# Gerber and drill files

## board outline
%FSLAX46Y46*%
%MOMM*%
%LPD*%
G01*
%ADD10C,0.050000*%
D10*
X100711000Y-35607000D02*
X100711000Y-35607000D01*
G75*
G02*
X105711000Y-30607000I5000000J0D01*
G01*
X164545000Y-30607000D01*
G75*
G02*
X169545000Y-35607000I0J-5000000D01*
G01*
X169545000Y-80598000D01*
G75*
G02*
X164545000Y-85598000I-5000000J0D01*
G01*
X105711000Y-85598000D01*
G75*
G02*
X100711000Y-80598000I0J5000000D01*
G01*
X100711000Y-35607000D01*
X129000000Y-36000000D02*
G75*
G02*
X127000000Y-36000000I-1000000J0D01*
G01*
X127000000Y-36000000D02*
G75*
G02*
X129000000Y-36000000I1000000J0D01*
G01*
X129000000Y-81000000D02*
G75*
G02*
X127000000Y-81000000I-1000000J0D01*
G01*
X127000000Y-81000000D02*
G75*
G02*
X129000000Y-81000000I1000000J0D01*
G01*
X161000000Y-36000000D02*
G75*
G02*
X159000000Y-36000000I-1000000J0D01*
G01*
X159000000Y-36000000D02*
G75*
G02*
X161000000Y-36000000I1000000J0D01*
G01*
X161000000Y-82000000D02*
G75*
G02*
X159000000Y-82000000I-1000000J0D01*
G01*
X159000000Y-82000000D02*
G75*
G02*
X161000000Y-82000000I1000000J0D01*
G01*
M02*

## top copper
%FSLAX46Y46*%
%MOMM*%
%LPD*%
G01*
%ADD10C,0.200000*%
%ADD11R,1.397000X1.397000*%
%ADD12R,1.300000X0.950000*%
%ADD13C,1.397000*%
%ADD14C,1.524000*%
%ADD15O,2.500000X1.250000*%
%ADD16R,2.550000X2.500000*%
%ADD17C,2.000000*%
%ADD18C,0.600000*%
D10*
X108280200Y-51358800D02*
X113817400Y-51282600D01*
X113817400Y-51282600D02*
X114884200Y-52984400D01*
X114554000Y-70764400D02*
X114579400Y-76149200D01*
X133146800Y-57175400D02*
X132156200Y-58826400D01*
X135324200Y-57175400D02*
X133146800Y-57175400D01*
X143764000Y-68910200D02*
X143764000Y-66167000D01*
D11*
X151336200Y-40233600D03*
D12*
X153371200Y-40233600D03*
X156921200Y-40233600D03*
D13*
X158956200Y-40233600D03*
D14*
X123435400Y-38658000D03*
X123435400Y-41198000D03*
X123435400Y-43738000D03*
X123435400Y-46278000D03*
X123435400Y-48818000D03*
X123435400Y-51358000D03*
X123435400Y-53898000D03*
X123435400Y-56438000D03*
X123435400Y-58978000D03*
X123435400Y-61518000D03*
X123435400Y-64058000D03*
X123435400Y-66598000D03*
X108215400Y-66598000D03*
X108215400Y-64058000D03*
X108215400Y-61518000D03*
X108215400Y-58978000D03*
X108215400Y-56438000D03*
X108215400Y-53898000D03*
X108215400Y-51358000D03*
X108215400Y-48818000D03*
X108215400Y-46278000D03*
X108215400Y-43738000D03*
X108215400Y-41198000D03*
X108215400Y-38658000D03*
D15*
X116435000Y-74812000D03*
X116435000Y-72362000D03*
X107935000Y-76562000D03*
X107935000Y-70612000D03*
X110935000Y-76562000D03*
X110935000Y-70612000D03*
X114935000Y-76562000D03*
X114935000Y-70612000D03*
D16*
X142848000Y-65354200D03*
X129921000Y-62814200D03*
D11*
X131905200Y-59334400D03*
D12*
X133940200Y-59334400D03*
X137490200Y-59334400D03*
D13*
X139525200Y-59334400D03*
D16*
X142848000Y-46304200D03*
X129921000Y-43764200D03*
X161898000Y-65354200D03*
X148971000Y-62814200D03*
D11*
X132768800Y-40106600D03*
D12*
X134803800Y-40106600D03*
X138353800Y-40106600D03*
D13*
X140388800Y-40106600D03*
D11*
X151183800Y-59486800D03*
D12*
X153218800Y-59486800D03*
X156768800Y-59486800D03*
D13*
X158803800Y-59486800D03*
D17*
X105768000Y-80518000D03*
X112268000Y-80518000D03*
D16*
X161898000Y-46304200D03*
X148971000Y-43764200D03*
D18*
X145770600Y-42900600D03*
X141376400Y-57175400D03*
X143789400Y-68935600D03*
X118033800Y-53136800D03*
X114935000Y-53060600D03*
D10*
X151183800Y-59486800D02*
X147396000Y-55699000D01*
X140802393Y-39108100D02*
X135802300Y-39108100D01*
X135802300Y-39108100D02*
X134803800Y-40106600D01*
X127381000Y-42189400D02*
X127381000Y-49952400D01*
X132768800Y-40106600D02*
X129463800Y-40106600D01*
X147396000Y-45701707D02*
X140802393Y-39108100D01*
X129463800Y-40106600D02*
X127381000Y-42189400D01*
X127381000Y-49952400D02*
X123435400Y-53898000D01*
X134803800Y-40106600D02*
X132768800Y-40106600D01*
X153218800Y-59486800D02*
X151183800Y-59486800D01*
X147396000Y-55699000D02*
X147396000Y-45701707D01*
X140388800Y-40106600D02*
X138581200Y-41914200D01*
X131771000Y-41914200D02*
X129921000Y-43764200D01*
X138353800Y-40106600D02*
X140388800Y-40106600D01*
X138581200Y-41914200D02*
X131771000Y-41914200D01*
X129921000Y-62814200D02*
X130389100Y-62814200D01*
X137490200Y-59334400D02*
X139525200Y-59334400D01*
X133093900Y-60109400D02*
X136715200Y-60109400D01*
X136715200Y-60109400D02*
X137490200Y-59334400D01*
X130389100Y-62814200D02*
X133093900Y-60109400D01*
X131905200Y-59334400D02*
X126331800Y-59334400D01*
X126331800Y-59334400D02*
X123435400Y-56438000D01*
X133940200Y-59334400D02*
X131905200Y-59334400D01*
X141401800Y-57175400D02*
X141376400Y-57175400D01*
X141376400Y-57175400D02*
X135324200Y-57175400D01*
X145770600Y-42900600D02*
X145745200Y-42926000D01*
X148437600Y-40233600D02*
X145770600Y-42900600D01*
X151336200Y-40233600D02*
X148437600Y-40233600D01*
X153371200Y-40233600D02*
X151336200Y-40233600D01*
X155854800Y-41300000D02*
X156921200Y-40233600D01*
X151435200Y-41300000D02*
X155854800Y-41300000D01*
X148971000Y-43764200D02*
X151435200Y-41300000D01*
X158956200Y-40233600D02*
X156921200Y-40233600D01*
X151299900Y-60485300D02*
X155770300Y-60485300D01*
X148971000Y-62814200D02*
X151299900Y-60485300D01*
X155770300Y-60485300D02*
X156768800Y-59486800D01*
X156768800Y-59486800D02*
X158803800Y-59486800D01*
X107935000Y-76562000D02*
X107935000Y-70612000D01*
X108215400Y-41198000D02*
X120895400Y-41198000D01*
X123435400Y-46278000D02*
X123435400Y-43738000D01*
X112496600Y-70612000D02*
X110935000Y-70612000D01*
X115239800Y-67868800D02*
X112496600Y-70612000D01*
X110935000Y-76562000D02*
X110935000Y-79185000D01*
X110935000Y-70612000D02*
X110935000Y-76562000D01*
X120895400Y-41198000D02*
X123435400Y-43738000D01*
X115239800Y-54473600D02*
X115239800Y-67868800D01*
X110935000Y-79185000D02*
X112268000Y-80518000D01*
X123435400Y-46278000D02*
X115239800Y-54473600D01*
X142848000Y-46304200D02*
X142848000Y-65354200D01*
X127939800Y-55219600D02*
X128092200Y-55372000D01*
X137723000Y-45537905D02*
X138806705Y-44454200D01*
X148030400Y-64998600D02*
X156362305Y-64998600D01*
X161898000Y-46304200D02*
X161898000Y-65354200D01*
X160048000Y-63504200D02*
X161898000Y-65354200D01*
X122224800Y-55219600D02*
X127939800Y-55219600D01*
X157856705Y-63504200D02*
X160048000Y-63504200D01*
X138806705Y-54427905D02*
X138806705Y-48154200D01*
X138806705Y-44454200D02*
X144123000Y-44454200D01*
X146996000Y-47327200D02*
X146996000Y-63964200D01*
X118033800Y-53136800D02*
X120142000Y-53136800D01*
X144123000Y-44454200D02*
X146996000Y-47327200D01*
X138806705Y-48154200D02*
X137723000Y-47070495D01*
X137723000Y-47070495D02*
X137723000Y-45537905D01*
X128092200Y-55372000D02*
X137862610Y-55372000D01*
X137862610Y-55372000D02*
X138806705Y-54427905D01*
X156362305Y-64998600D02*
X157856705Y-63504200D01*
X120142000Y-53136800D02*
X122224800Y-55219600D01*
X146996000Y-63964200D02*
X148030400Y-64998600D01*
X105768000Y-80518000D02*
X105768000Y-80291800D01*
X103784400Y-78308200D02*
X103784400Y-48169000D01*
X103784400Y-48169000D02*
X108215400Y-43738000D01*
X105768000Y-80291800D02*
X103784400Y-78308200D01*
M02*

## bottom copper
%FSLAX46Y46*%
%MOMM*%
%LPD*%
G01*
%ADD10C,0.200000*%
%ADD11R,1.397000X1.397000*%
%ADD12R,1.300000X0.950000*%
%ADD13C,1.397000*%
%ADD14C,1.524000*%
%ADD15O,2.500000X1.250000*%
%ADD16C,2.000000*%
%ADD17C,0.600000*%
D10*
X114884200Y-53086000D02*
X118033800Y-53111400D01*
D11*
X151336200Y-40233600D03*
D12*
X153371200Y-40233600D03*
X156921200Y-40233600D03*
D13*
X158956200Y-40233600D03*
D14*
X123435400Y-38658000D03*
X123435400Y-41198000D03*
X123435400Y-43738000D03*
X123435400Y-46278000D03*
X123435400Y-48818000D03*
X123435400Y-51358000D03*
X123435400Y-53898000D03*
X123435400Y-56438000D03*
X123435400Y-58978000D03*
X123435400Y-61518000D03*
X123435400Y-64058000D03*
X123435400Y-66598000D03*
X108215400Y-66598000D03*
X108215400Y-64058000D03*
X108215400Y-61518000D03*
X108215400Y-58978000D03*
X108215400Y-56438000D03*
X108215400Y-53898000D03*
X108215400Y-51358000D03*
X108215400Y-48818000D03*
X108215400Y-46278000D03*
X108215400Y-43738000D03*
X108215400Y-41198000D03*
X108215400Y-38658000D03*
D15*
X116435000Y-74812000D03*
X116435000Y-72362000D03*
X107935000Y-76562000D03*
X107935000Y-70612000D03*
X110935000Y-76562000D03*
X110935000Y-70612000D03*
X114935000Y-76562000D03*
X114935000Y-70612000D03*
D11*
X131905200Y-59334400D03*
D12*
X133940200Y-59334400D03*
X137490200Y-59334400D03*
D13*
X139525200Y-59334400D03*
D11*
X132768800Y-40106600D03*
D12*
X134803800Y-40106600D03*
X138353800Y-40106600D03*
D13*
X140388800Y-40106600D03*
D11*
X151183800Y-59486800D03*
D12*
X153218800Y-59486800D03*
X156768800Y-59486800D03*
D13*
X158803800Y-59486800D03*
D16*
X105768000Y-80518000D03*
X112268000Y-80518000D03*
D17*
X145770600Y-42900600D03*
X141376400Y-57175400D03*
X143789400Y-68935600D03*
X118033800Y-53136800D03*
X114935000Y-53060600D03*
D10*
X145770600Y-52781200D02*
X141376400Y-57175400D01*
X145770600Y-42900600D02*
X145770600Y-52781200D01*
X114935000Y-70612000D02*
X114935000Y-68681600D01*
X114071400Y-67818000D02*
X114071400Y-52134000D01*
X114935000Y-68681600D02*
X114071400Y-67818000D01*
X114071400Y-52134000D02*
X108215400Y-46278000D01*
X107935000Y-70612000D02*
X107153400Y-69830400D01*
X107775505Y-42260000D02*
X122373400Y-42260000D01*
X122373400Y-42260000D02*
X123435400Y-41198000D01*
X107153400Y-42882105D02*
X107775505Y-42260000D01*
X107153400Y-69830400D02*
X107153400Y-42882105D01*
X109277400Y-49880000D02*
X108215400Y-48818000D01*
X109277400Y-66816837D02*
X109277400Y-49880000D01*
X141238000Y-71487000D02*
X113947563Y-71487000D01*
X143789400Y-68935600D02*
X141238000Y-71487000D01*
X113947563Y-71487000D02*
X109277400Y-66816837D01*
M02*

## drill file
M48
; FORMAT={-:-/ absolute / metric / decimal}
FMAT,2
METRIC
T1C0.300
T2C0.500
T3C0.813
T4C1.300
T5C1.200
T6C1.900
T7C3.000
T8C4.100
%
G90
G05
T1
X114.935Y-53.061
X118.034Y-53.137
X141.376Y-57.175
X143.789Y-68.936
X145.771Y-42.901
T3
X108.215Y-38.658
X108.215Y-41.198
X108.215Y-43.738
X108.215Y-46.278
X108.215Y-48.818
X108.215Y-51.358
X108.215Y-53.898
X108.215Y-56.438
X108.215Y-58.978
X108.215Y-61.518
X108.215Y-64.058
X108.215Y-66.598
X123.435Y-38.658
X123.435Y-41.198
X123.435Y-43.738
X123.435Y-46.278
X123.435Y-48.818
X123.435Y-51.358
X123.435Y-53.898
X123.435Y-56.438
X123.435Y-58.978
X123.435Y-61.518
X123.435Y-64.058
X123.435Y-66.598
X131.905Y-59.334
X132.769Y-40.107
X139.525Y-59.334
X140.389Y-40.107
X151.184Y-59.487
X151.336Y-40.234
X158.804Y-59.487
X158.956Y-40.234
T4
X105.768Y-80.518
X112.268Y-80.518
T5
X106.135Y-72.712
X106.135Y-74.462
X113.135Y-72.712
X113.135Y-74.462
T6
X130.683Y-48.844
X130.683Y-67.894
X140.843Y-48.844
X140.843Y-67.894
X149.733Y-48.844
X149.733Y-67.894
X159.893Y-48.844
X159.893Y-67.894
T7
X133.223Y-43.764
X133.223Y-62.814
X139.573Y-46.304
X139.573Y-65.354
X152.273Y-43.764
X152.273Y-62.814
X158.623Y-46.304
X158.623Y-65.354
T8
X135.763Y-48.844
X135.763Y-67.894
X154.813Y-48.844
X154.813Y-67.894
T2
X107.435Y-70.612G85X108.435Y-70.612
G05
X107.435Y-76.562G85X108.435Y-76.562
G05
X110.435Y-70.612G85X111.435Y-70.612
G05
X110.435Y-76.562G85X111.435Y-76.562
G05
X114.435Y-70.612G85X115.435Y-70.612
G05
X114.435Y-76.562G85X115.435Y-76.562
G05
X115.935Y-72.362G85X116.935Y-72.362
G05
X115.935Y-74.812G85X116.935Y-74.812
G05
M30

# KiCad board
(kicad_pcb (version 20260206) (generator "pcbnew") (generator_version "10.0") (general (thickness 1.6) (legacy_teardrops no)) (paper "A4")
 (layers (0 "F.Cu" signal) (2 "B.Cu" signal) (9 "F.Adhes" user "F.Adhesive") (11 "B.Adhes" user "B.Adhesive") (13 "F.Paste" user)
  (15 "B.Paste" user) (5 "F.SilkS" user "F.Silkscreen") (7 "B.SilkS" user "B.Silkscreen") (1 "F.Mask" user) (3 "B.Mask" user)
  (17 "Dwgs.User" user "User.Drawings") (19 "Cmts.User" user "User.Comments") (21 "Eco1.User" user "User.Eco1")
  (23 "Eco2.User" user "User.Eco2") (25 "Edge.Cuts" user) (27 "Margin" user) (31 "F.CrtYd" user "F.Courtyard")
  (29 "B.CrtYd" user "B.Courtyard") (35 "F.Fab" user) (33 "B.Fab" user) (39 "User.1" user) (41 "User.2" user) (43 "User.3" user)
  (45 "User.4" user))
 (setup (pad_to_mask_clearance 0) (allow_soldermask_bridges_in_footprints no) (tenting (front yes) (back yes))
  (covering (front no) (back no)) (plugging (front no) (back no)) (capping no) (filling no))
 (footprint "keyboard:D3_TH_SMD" (layer "F.Cu") (at 155.1462 40.2336)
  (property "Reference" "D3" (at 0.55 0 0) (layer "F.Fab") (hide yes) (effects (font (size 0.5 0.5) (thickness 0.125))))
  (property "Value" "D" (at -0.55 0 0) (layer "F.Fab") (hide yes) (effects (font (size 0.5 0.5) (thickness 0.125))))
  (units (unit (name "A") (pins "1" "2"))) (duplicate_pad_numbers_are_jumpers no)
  (pad "1" thru_hole rect (at -3.81 0) (size 1.397 1.397) (drill 0.8128) (layers "*.Cu" "*.Mask" "F.SilkS") (remove_unused_layers no)
   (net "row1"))
  (pad "1" smd rect (at -1.775 0) (size 1.3 0.95) (layers "F.Cu" "F.Mask" "F.Paste") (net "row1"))
  (pad "1" smd rect (at -1.775 0) (size 1.3 0.95) (layers "B.Cu" "B.Mask" "B.Paste") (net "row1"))
  (pad "2" smd rect (at 1.775 0) (size 1.3 0.95) (layers "F.Cu" "F.Mask" "F.Paste") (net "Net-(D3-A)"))
  (pad "2" smd rect (at 1.775 0) (size 1.3 0.95) (layers "B.Cu" "B.Mask" "B.Paste") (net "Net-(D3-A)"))
  (pad "2" thru_hole circle (at 3.81 0) (size 1.397 1.397) (drill 0.8128) (layers "*.Cu" "*.Mask" "F.SilkS") (remove_unused_layers no)
   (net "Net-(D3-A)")))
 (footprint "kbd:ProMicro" (layer "F.Cu") (at 115.824 53.136)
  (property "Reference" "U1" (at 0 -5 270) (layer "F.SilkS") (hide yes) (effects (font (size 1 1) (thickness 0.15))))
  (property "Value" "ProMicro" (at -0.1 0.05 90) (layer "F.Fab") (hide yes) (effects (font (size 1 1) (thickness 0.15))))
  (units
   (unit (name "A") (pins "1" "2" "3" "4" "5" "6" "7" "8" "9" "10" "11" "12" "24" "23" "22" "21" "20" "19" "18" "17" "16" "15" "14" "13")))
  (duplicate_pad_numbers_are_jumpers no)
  (pad "1" thru_hole circle (at 7.6114 -14.478) (size 1.524 1.524) (drill 0.8128) (layers "*.Cu" "B.Mask") (remove_unused_layers no)
   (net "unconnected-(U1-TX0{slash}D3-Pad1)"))
  (pad "2" thru_hole circle (at 7.6114 -11.938) (size 1.524 1.524) (drill 0.8128) (layers "*.Cu" "B.Mask") (remove_unused_layers no)
   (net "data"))
  (pad "3" thru_hole circle (at 7.6114 -9.398) (size 1.524 1.524) (drill 0.8128) (layers "*.Cu" "B.Mask") (remove_unused_layers no)
   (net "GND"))
  (pad "4" thru_hole circle (at 7.6114 -6.858) (size 1.524 1.524) (drill 0.8128) (layers "*.Cu" "B.Mask") (remove_unused_layers no)
   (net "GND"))
  (pad "5" thru_hole circle (at 7.6114 -4.318) (size 1.524 1.524) (drill 0.8128) (layers "*.Cu" "B.Mask") (remove_unused_layers no)
   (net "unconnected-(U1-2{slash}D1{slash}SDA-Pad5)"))
  (pad "6" thru_hole circle (at 7.6114 -1.778) (size 1.524 1.524) (drill 0.8128) (layers "*.Cu" "B.Mask") (remove_unused_layers no)
   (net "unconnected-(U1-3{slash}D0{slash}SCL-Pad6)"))
  (pad "7" thru_hole circle (at 7.6114 0.762) (size 1.524 1.524) (drill 0.8128) (layers "*.Cu" "B.Mask") (remove_unused_layers no)
   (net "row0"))
  (pad "8" thru_hole circle (at 7.6114 3.302) (size 1.524 1.524) (drill 0.8128) (layers "*.Cu" "B.Mask") (remove_unused_layers no)
   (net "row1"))
  (pad "9" thru_hole circle (at 7.6114 5.842) (size 1.524 1.524) (drill 0.8128) (layers "*.Cu" "B.Mask") (remove_unused_layers no)
   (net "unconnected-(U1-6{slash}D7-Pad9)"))
  (pad "10" thru_hole circle (at 7.6114 8.382) (size 1.524 1.524) (drill 0.8128) (layers "*.Cu" "B.Mask") (remove_unused_layers no)
   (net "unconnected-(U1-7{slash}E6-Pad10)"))
  (pad "11" thru_hole circle (at 7.6114 10.922) (size 1.524 1.524) (drill 0.8128) (layers "*.Cu" "B.Mask") (remove_unused_layers no)
   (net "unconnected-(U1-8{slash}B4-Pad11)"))
  (pad "12" thru_hole circle (at 7.6114 13.462) (size 1.524 1.524) (drill 0.8128) (layers "*.Cu" "B.Mask") (remove_unused_layers no)
   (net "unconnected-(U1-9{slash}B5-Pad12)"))
  (pad "13" thru_hole circle (at -7.6086 13.462) (size 1.524 1.524) (drill 0.8128) (layers "*.Cu" "B.Mask") (remove_unused_layers no)
   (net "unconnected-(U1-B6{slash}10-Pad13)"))
  (pad "14" thru_hole circle (at -7.6086 10.922) (size 1.524 1.524) (drill 0.8128) (layers "*.Cu" "B.Mask") (remove_unused_layers no)
   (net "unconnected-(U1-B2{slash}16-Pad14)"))
  (pad "15" thru_hole circle (at -7.6086 8.382) (size 1.524 1.524) (drill 0.8128) (layers "*.Cu" "B.Mask") (remove_unused_layers no)
   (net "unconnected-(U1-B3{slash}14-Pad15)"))
  (pad "16" thru_hole circle (at -7.6086 5.842) (size 1.524 1.524) (drill 0.8128) (layers "*.Cu" "B.Mask") (remove_unused_layers no)
   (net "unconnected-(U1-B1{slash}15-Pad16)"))
  (pad "17" thru_hole circle (at -7.6086 3.302) (size 1.524 1.524) (drill 0.8128) (layers "*.Cu" "B.Mask") (remove_unused_layers no)
   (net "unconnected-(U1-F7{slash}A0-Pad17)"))
  (pad "18" thru_hole circle (at -7.6086 0.762) (size 1.524 1.524) (drill 0.8128) (layers "*.Cu" "B.Mask") (remove_unused_layers no)
   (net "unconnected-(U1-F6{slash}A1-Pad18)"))
  (pad "19" thru_hole circle (at -7.6086 -1.778) (size 1.524 1.524) (drill 0.8128) (layers "*.Cu" "B.Mask") (remove_unused_layers no)
   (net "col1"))
  (pad "20" thru_hole circle (at -7.6086 -4.318) (size 1.524 1.524) (drill 0.8128) (layers "*.Cu" "B.Mask") (remove_unused_layers no)
   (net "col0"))
  (pad "21" thru_hole circle (at -7.6086 -6.858) (size 1.524 1.524) (drill 0.8128) (layers "*.Cu" "B.Mask") (remove_unused_layers no)
   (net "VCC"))
  (pad "22" thru_hole circle (at -7.6086 -9.398) (size 1.524 1.524) (drill 0.8128) (layers "*.Cu" "B.Mask") (remove_unused_layers no)
   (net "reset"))
  (pad "23" thru_hole circle (at -7.6086 -11.938) (size 1.524 1.524) (drill 0.8128) (layers "*.Cu" "B.Mask") (remove_unused_layers no)
   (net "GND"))
  (pad "24" thru_hole circle (at -7.6086 -14.478) (size 1.524 1.524) (drill 0.8128) (layers "*.Cu" "B.Mask") (remove_unused_layers no)
   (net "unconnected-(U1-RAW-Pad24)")))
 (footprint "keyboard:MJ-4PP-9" (layer "F.Cu") (at 104.635 72.712 90)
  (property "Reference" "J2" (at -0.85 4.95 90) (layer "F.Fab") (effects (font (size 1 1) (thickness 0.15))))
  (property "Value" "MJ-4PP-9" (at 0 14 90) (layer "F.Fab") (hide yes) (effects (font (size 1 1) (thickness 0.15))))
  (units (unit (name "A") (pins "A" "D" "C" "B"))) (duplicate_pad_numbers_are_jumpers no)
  (pad "" np_thru_hole circle (at -1.75 1.5 90) (size 1.2 1.2) (drill 1.2) (layers "*.Cu" "*.Mask" "F.SilkS"))
  (pad "" np_thru_hole circle (at -1.75 8.5 90) (size 1.2 1.2) (drill 1.2) (layers "*.Cu" "*.Mask" "F.SilkS"))
  (pad "" np_thru_hole circle (at 0 1.5 90) (size 1.2 1.2) (drill 1.2) (layers "*.Cu" "*.Mask" "F.SilkS"))
  (pad "" np_thru_hole circle (at 0 8.5 90) (size 1.2 1.2) (drill 1.2) (layers "*.Cu" "*.Mask" "F.SilkS"))
  (pad "A" thru_hole oval (at -2.1 11.8 90) (size 1.25 2.5) (drill oval 0.5 1.5) (layers "*.Cu" "B.Mask" "F.SilkS")
   (remove_unused_layers no) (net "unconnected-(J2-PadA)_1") (clearance 0.15))
  (pad "A" thru_hole oval (at 0.35 11.8 90) (size 1.25 2.5) (drill oval 0.5 1.5) (layers "*.Cu" "F.Mask" "B.SilkS")
   (remove_unused_layers no) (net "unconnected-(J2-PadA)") (clearance 0.15))
  (pad "B" thru_hole oval (at -3.85 3.3 90) (size 1.25 2.5) (drill oval 0.5 1.5) (layers "*.Cu" "F.Mask" "B.SilkS")
   (remove_unused_layers no) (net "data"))
  (pad "B" thru_hole oval (at 2.1 3.3 90) (size 1.25 2.5) (drill oval 0.5 1.5) (layers "*.Cu" "B.Mask" "F.SilkS") (remove_unused_layers no)
   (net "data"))
  (pad "C" thru_hole oval (at -3.85 6.3 90) (size 1.25 2.5) (drill oval 0.5 1.5) (layers "*.Cu" "F.Mask" "B.SilkS")
   (remove_unused_layers no) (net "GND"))
  (pad "C" thru_hole oval (at 2.1 6.3 90) (size 1.25 2.5) (drill oval 0.5 1.5) (layers "*.Cu" "B.Mask" "F.SilkS") (remove_unused_layers no)
   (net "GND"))
  (pad "D" thru_hole oval (at -3.85 10.3 90) (size 1.25 2.5) (drill oval 0.5 1.5) (layers "*.Cu" "F.Mask" "B.SilkS")
   (remove_unused_layers no) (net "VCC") (clearance 0.15))
  (pad "D" thru_hole oval (at 2.1 10.3 90) (size 1.25 2.5) (drill oval 0.5 1.5) (layers "*.Cu" "B.Mask" "F.SilkS") (remove_unused_layers no)
   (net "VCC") (clearance 0.15)))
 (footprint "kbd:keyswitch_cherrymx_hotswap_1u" (layer "F.Cu") (at 135.763 67.8942)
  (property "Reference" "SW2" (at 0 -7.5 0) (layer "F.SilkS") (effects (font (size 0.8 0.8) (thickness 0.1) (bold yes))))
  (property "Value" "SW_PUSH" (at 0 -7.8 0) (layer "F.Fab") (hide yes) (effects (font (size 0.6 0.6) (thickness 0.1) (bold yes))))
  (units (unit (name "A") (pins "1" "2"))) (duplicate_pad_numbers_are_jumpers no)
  (pad "" np_thru_hole circle (at -5.08 0) (size 1.9 1.9) (drill 1.9) (layers "*.Cu" "*.Mask"))
  (pad "" np_thru_hole circle (at -2.54 -5.08) (size 3 3) (drill 3) (layers "*.Cu" "*.Mask"))
  (pad "" np_thru_hole circle (at 0 0 270) (size 4.1 4.1) (drill 4.1) (layers "*.Cu" "*.Mask"))
  (pad "" np_thru_hole circle (at 3.81 -2.54) (size 3 3) (drill 3) (layers "*.Cu" "*.Mask"))
  (pad "" np_thru_hole circle (at 5.08 0) (size 1.9 1.9) (drill 1.9) (layers "*.Cu" "*.Mask"))
  (pad "1" smd rect (at 7.085 -2.54 180) (size 2.55 2.5) (layers "F.Cu" "F.Mask" "F.Paste") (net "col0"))
  (pad "2" smd rect (at -5.842 -5.08 180) (size 2.55 2.5) (layers "F.Cu" "F.Mask" "F.Paste") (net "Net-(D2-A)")))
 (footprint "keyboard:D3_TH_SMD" (layer "F.Cu") (at 135.7152 59.3344)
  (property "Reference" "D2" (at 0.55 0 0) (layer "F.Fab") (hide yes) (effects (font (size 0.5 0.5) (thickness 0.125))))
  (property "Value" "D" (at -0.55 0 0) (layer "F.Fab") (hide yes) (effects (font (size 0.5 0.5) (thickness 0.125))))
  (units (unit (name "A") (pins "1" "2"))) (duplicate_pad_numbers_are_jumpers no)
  (pad "1" thru_hole rect (at -3.81 0) (size 1.397 1.397) (drill 0.8128) (layers "*.Cu" "*.Mask" "F.SilkS") (remove_unused_layers no)
   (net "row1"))
  (pad "1" smd rect (at -1.775 0) (size 1.3 0.95) (layers "F.Cu" "F.Mask" "F.Paste") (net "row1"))
  (pad "1" smd rect (at -1.775 0) (size 1.3 0.95) (layers "B.Cu" "B.Mask" "B.Paste") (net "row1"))
  (pad "2" smd rect (at 1.775 0) (size 1.3 0.95) (layers "F.Cu" "F.Mask" "F.Paste") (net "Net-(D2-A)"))
  (pad "2" smd rect (at 1.775 0) (size 1.3 0.95) (layers "B.Cu" "B.Mask" "B.Paste") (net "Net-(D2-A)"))
  (pad "2" thru_hole circle (at 3.81 0) (size 1.397 1.397) (drill 0.8128) (layers "*.Cu" "*.Mask" "F.SilkS") (remove_unused_layers no)
   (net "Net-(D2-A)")))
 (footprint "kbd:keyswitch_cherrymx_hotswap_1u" (layer "F.Cu") (at 135.763 48.8442)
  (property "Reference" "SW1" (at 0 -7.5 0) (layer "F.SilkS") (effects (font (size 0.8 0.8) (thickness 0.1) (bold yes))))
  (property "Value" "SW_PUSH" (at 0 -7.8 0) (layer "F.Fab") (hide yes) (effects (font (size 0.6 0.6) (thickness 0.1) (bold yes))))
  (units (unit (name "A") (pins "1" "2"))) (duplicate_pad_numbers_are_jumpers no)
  (pad "" np_thru_hole circle (at -5.08 0) (size 1.9 1.9) (drill 1.9) (layers "*.Cu" "*.Mask"))
  (pad "" np_thru_hole circle (at -2.54 -5.08) (size 3 3) (drill 3) (layers "*.Cu" "*.Mask"))
  (pad "" np_thru_hole circle (at 0 0 270) (size 4.1 4.1) (drill 4.1) (layers "*.Cu" "*.Mask"))
  (pad "" np_thru_hole circle (at 3.81 -2.54) (size 3 3) (drill 3) (layers "*.Cu" "*.Mask"))
  (pad "" np_thru_hole circle (at 5.08 0) (size 1.9 1.9) (drill 1.9) (layers "*.Cu" "*.Mask"))
  (pad "1" smd rect (at 7.085 -2.54 180) (size 2.55 2.5) (layers "F.Cu" "F.Mask" "F.Paste") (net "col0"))
  (pad "2" smd rect (at -5.842 -5.08 180) (size 2.55 2.5) (layers "F.Cu" "F.Mask" "F.Paste") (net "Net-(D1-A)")))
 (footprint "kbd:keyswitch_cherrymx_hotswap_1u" (layer "F.Cu") (at 154.813 67.8942)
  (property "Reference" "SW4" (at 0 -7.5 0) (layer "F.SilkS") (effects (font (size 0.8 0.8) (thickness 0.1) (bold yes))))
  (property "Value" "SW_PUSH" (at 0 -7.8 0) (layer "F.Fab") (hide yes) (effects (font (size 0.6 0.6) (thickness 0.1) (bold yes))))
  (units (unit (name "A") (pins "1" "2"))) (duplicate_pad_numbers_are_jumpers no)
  (pad "" np_thru_hole circle (at -5.08 0) (size 1.9 1.9) (drill 1.9) (layers "*.Cu" "*.Mask"))
  (pad "" np_thru_hole circle (at -2.54 -5.08) (size 3 3) (drill 3) (layers "*.Cu" "*.Mask"))
  (pad "" np_thru_hole circle (at 0 0 270) (size 4.1 4.1) (drill 4.1) (layers "*.Cu" "*.Mask"))
  (pad "" np_thru_hole circle (at 3.81 -2.54) (size 3 3) (drill 3) (layers "*.Cu" "*.Mask"))
  (pad "" np_thru_hole circle (at 5.08 0) (size 1.9 1.9) (drill 1.9) (layers "*.Cu" "*.Mask"))
  (pad "1" smd rect (at 7.085 -2.54 180) (size 2.55 2.5) (layers "F.Cu" "F.Mask" "F.Paste") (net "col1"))
  (pad "2" smd rect (at -5.842 -5.08 180) (size 2.55 2.5) (layers "F.Cu" "F.Mask" "F.Paste") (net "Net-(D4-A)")))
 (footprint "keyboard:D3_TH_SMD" (layer "F.Cu") (at 136.5788 40.1066)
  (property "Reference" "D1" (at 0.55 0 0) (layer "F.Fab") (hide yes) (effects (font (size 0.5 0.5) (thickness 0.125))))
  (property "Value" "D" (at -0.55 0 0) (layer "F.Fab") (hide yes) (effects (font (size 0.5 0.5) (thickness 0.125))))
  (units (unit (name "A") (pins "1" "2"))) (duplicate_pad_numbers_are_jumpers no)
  (pad "1" thru_hole rect (at -3.81 0) (size 1.397 1.397) (drill 0.8128) (layers "*.Cu" "*.Mask" "F.SilkS") (remove_unused_layers no)
   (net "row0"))
  (pad "1" smd rect (at -1.775 0) (size 1.3 0.95) (layers "F.Cu" "F.Mask" "F.Paste") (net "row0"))
  (pad "1" smd rect (at -1.775 0) (size 1.3 0.95) (layers "B.Cu" "B.Mask" "B.Paste") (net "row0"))
  (pad "2" smd rect (at 1.775 0) (size 1.3 0.95) (layers "F.Cu" "F.Mask" "F.Paste") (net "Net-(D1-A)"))
  (pad "2" smd rect (at 1.775 0) (size 1.3 0.95) (layers "B.Cu" "B.Mask" "B.Paste") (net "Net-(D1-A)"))
  (pad "2" thru_hole circle (at 3.81 0) (size 1.397 1.397) (drill 0.8128) (layers "*.Cu" "*.Mask" "F.SilkS") (remove_unused_layers no)
   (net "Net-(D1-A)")))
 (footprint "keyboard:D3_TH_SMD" (layer "F.Cu") (at 154.9938 59.4868)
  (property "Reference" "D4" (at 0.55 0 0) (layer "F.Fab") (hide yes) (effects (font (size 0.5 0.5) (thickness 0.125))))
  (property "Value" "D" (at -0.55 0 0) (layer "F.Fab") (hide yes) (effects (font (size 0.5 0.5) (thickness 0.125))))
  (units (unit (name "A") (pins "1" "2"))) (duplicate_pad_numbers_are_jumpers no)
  (pad "1" thru_hole rect (at -3.81 0) (size 1.397 1.397) (drill 0.8128) (layers "*.Cu" "*.Mask" "F.SilkS") (remove_unused_layers no)
   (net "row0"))
  (pad "1" smd rect (at -1.775 0) (size 1.3 0.95) (layers "F.Cu" "F.Mask" "F.Paste") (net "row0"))
  (pad "1" smd rect (at -1.775 0) (size 1.3 0.95) (layers "B.Cu" "B.Mask" "B.Paste") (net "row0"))
  (pad "2" smd rect (at 1.775 0) (size 1.3 0.95) (layers "F.Cu" "F.Mask" "F.Paste") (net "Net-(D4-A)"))
  (pad "2" smd rect (at 1.775 0) (size 1.3 0.95) (layers "B.Cu" "B.Mask" "B.Paste") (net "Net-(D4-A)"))
  (pad "2" thru_hole circle (at 3.81 0) (size 1.397 1.397) (drill 0.8128) (layers "*.Cu" "*.Mask" "F.SilkS") (remove_unused_layers no)
   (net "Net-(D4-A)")))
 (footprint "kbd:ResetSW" (layer "F.Cu") (at 109.018 80.518 180)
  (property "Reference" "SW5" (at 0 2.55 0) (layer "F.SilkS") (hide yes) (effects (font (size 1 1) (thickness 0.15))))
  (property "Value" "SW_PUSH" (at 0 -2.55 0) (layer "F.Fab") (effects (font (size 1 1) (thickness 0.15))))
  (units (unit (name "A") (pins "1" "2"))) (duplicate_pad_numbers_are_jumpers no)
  (pad "1" thru_hole circle (at 3.25 0 180) (size 2 2) (drill 1.3) (layers "*.Cu" "B.Mask") (remove_unused_layers no) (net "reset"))
  (pad "2" thru_hole circle (at -3.25 0 180) (size 2 2) (drill 1.3) (layers "*.Cu" "B.Mask") (remove_unused_layers no) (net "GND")))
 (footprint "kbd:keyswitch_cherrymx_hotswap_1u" (layer "F.Cu") (at 154.813 48.8442)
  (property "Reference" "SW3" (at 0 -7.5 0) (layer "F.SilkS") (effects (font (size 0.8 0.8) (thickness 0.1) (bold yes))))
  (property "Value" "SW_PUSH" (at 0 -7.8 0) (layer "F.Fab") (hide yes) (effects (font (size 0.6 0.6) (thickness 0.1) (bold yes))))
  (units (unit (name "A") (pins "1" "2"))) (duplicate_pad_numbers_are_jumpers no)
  (pad "" np_thru_hole circle (at -5.08 0) (size 1.9 1.9) (drill 1.9) (layers "*.Cu" "*.Mask"))
  (pad "" np_thru_hole circle (at -2.54 -5.08) (size 3 3) (drill 3) (layers "*.Cu" "*.Mask"))
  (pad "" np_thru_hole circle (at 0 0 270) (size 4.1 4.1) (drill 4.1) (layers "*.Cu" "*.Mask"))
  (pad "" np_thru_hole circle (at 3.81 -2.54) (size 3 3) (drill 3) (layers "*.Cu" "*.Mask"))
  (pad "" np_thru_hole circle (at 5.08 0) (size 1.9 1.9) (drill 1.9) (layers "*.Cu" "*.Mask"))
  (pad "1" smd rect (at 7.085 -2.54 180) (size 2.55 2.5) (layers "F.Cu" "F.Mask" "F.Paste") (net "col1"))
  (pad "2" smd rect (at -5.842 -5.08 180) (size 2.55 2.5) (layers "F.Cu" "F.Mask" "F.Paste") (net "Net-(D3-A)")))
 (gr_line (start 108.2802 51.3588) (end 113.8174 51.2826) (stroke (width 0.2) (type default)) (layer "F.Cu") (net "col1"))
 (gr_line (start 113.8174 51.2826) (end 114.8842 52.9844) (stroke (width 0.2) (type default)) (layer "F.Cu") (net "col1"))
 (gr_line (start 114.554 70.7644) (end 114.5794 76.1492) (stroke (width 0.2) (type default)) (layer "F.Cu") (net "VCC"))
 (gr_line (start 133.1468 57.1754) (end 132.1562 58.8264) (stroke (width 0.2) (type default)) (layer "F.Cu") (net "row1"))
 (gr_line (start 135.3242 57.1754) (end 133.1468 57.1754) (stroke (width 0.2) (type default)) (layer "F.Cu") (net "row1"))
 (gr_line (start 143.764 68.9102) (end 143.764 66.167) (stroke (width 0.2) (type default)) (layer "F.Cu") (net "col0"))
 (gr_line (start 114.8842 53.086) (end 118.0338 53.1114) (stroke (width 0.2) (type default)) (layer "B.Cu") (net "col1"))
 (gr_rect (start 100.711 30.607) (end 169.545 85.598) (radius 5) (stroke (width 0.05) (type solid)) (fill no) (layer "Edge.Cuts"))
 (gr_circle (center 128 36) (end 127 36) (stroke (width 0.05) (type default)) (fill no) (layer "Edge.Cuts"))
 (gr_circle (center 128 81) (end 127 81) (stroke (width 0.05) (type default)) (fill no) (layer "Edge.Cuts"))
 (gr_circle (center 160 36) (end 161 36) (stroke (width 0.05) (type default)) (fill no) (layer "Edge.Cuts"))
 (gr_circle (center 160 82) (end 161 82) (stroke (width 0.05) (type default)) (fill no) (layer "Edge.Cuts"))
 (segment (start 151.1838 59.4868) (end 147.396 55.699) (width 0.2) (layer "F.Cu") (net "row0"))
 (segment (start 140.802393 39.1081) (end 135.8023 39.1081) (width 0.2) (layer "F.Cu") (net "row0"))
 (segment (start 135.8023 39.1081) (end 134.8038 40.1066) (width 0.2) (layer "F.Cu") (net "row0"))
 (segment (start 127.381 42.1894) (end 127.381 49.9524) (width 0.2) (layer "F.Cu") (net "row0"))
 (segment (start 132.7688 40.1066) (end 129.4638 40.1066) (width 0.2) (layer "F.Cu") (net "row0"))
 (segment (start 147.396 45.701707) (end 140.802393 39.1081) (width 0.2) (layer "F.Cu") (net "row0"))
 (segment (start 129.4638 40.1066) (end 127.381 42.1894) (width 0.2) (layer "F.Cu") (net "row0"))
 (segment (start 127.381 49.9524) (end 123.4354 53.898) (width 0.2) (layer "F.Cu") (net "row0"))
 (segment (start 134.8038 40.1066) (end 132.7688 40.1066) (width 0.2) (layer "F.Cu") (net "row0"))
 (segment (start 153.2188 59.4868) (end 151.1838 59.4868) (width 0.2) (layer "F.Cu") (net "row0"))
 (segment (start 147.396 55.699) (end 147.396 45.701707) (width 0.2) (layer "F.Cu") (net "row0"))
 (segment (start 140.3888 40.1066) (end 138.5812 41.9142) (width 0.2) (layer "F.Cu") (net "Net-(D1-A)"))
 (segment (start 131.771 41.9142) (end 129.921 43.7642) (width 0.2) (layer "F.Cu") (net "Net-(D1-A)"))
 (segment (start 138.3538 40.1066) (end 140.3888 40.1066) (width 0.2) (layer "F.Cu") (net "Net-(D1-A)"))
 (segment (start 138.5812 41.9142) (end 131.771 41.9142) (width 0.2) (layer "F.Cu") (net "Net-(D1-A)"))
 (segment (start 129.921 62.8142) (end 130.3891 62.8142) (width 0.2) (layer "F.Cu") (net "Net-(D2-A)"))
 (segment (start 137.4902 59.3344) (end 139.5252 59.3344) (width 0.2) (layer "F.Cu") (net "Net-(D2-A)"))
 (segment (start 133.0939 60.1094) (end 136.7152 60.1094) (width 0.2) (layer "F.Cu") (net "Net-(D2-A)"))
 (segment (start 136.7152 60.1094) (end 137.4902 59.3344) (width 0.2) (layer "F.Cu") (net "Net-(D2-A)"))
 (segment (start 130.3891 62.8142) (end 133.0939 60.1094) (width 0.2) (layer "F.Cu") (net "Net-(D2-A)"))
 (segment (start 131.9052 59.3344) (end 126.3318 59.3344) (width 0.2) (layer "F.Cu") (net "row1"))
 (segment (start 126.3318 59.3344) (end 123.4354 56.438) (width 0.2) (layer "F.Cu") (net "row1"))
 (segment (start 133.9402 59.3344) (end 131.9052 59.3344) (width 0.2) (layer "F.Cu") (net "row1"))
 (segment (start 141.4018 57.1754) (end 141.3764 57.1754) (width 0.2) (layer "F.Cu") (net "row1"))
 (segment (start 141.3764 57.1754) (end 135.3242 57.1754) (width 0.2) (layer "F.Cu") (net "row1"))
 (segment (start 145.7706 42.9006) (end 145.7452 42.926) (width 0.2) (layer "F.Cu") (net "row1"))
 (segment (start 148.4376 40.2336) (end 145.7706 42.9006) (width 0.2) (layer "F.Cu") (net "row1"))
 (segment (start 151.3362 40.2336) (end 148.4376 40.2336) (width 0.2) (layer "F.Cu") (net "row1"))
 (segment (start 153.3712 40.2336) (end 151.3362 40.2336) (width 0.2) (layer "F.Cu") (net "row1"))
 (via (at 145.7706 42.9006) (size 0.6) (drill 0.3) (layers "F.Cu" "B.Cu") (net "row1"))
 (via (at 141.3764 57.1754) (size 0.6) (drill 0.3) (layers "F.Cu" "B.Cu") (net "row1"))
 (segment (start 145.7706 52.7812) (end 141.3764 57.1754) (width 0.2) (layer "B.Cu") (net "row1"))
 (segment (start 145.7706 42.9006) (end 145.7706 52.7812) (width 0.2) (layer "B.Cu") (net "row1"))
 (segment (start 155.8548 41.3) (end 156.9212 40.2336) (width 0.2) (layer "F.Cu") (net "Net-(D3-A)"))
 (segment (start 151.4352 41.3) (end 155.8548 41.3) (width 0.2) (layer "F.Cu") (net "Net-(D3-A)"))
 (segment (start 148.971 43.7642) (end 151.4352 41.3) (width 0.2) (layer "F.Cu") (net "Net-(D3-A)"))
 (segment (start 158.9562 40.2336) (end 156.9212 40.2336) (width 0.2) (layer "F.Cu") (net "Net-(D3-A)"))
 (segment (start 151.2999 60.4853) (end 155.7703 60.4853) (width 0.2) (layer "F.Cu") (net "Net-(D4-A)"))
 (segment (start 148.971 62.8142) (end 151.2999 60.4853) (width 0.2) (layer "F.Cu") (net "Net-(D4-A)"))
 (segment (start 155.7703 60.4853) (end 156.7688 59.4868) (width 0.2) (layer "F.Cu") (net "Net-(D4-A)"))
 (segment (start 156.7688 59.4868) (end 158.8038 59.4868) (width 0.2) (layer "F.Cu") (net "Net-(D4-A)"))
 (segment (start 114.935 70.612) (end 114.935 68.6816) (width 0.2) (layer "B.Cu") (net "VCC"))
 (segment (start 114.0714 67.818) (end 114.0714 52.134) (width 0.2) (layer "B.Cu") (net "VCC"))
 (segment (start 114.935 68.6816) (end 114.0714 67.818) (width 0.2) (layer "B.Cu") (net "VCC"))
 (segment (start 114.0714 52.134) (end 108.2154 46.278) (width 0.2) (layer "B.Cu") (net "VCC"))
 (segment (start 107.935 76.562) (end 107.935 70.612) (width 0.2) (layer "F.Cu") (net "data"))
 (segment (start 107.935 70.612) (end 107.1534 69.8304) (width 0.2) (layer "B.Cu") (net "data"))
 (segment (start 107.775505 42.26) (end 122.3734 42.26) (width 0.2) (layer "B.Cu") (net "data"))
 (segment (start 122.3734 42.26) (end 123.4354 41.198) (width 0.2) (layer "B.Cu") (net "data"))
 (segment (start 107.1534 42.882105) (end 107.775505 42.26) (width 0.2) (layer "B.Cu") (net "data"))
 (segment (start 107.1534 69.8304) (end 107.1534 42.882105) (width 0.2) (layer "B.Cu") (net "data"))
 (segment (start 108.2154 41.198) (end 120.8954 41.198) (width 0.2) (layer "F.Cu") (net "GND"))
 (segment (start 123.4354 46.278) (end 123.4354 43.738) (width 0.2) (layer "F.Cu") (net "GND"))
 (segment (start 112.4966 70.612) (end 110.935 70.612) (width 0.2) (layer "F.Cu") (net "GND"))
 (segment (start 115.2398 67.8688) (end 112.4966 70.612) (width 0.2) (layer "F.Cu") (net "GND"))
 (segment (start 110.935 76.562) (end 110.935 79.185) (width 0.2) (layer "F.Cu") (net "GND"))
 (segment (start 110.935 70.612) (end 110.935 76.562) (width 0.2) (layer "F.Cu") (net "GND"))
 (segment (start 120.8954 41.198) (end 123.4354 43.738) (width 0.2) (layer "F.Cu") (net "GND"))
 (segment (start 115.2398 54.4736) (end 115.2398 67.8688) (width 0.2) (layer "F.Cu") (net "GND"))
 (segment (start 110.935 79.185) (end 112.268 80.518) (width 0.2) (layer "F.Cu") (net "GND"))
 (segment (start 123.4354 46.278) (end 115.2398 54.4736) (width 0.2) (layer "F.Cu") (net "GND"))
 (segment (start 142.848 46.3042) (end 142.848 65.3542) (width 0.2) (layer "F.Cu") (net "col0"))
 (via (at 143.7894 68.9356) (size 0.6) (drill 0.3) (layers "F.Cu" "B.Cu") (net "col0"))
 (segment (start 109.2774 49.88) (end 108.2154 48.818) (width 0.2) (layer "B.Cu") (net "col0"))
 (segment (start 109.2774 66.816837) (end 109.2774 49.88) (width 0.2) (layer "B.Cu") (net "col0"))
 (segment (start 141.238 71.487) (end 113.947563 71.487) (width 0.2) (layer "B.Cu") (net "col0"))
 (segment (start 143.7894 68.9356) (end 141.238 71.487) (width 0.2) (layer "B.Cu") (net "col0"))
 (segment (start 113.947563 71.487) (end 109.2774 66.816837) (width 0.2) (layer "B.Cu") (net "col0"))
 (segment (start 127.9398 55.2196) (end 128.0922 55.372) (width 0.2) (layer "F.Cu") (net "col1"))
 (segment (start 137.723 45.537905) (end 138.806705 44.4542) (width 0.2) (layer "F.Cu") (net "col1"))
 (segment (start 148.0304 64.9986) (end 156.362305 64.9986) (width 0.2) (layer "F.Cu") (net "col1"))
 (segment (start 161.898 46.3042) (end 161.898 65.3542) (width 0.2) (layer "F.Cu") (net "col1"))
 (segment (start 160.048 63.5042) (end 161.898 65.3542) (width 0.2) (layer "F.Cu") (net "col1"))
 (segment (start 122.2248 55.2196) (end 127.9398 55.2196) (width 0.2) (layer "F.Cu") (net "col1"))
 (segment (start 157.856705 63.5042) (end 160.048 63.5042) (width 0.2) (layer "F.Cu") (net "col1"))
 (segment (start 138.806705 54.427905) (end 138.806705 48.1542) (width 0.2) (layer "F.Cu") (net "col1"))
 (segment (start 138.806705 44.4542) (end 144.123 44.4542) (width 0.2) (layer "F.Cu") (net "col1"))
 (segment (start 146.996 47.3272) (end 146.996 63.9642) (width 0.2) (layer "F.Cu") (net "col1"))
 (segment (start 118.0338 53.1368) (end 120.142 53.1368) (width 0.2) (layer "F.Cu") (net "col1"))
 (segment (start 144.123 44.4542) (end 146.996 47.3272) (width 0.2) (layer "F.Cu") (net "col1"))
 (segment (start 138.806705 48.1542) (end 137.723 47.070495) (width 0.2) (layer "F.Cu") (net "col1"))
 (segment (start 137.723 47.070495) (end 137.723 45.537905) (width 0.2) (layer "F.Cu") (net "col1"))
 (segment (start 128.0922 55.372) (end 137.86261 55.372) (width 0.2) (layer "F.Cu") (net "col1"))
 (segment (start 137.86261 55.372) (end 138.806705 54.427905) (width 0.2) (layer "F.Cu") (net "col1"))
 (segment (start 156.362305 64.9986) (end 157.856705 63.5042) (width 0.2) (layer "F.Cu") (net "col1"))
 (segment (start 120.142 53.1368) (end 122.2248 55.2196) (width 0.2) (layer "F.Cu") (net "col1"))
 (segment (start 146.996 63.9642) (end 148.0304 64.9986) (width 0.2) (layer "F.Cu") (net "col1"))
 (via (at 118.0338 53.1368) (size 0.6) (drill 0.3) (layers "F.Cu" "B.Cu") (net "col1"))
 (via (at 114.935 53.0606) (size 0.6) (drill 0.3) (layers "F.Cu" "B.Cu") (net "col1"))
 (segment (start 105.768 80.518) (end 105.768 80.2918) (width 0.2) (layer "F.Cu") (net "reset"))
 (segment (start 103.7844 78.3082) (end 103.7844 48.169) (width 0.2) (layer "F.Cu") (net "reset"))
 (segment (start 103.7844 48.169) (end 108.2154 43.738) (width 0.2) (layer "F.Cu") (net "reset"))
 (segment (start 105.768 80.2918) (end 103.7844 78.3082) (width 0.2) (layer "F.Cu") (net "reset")))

